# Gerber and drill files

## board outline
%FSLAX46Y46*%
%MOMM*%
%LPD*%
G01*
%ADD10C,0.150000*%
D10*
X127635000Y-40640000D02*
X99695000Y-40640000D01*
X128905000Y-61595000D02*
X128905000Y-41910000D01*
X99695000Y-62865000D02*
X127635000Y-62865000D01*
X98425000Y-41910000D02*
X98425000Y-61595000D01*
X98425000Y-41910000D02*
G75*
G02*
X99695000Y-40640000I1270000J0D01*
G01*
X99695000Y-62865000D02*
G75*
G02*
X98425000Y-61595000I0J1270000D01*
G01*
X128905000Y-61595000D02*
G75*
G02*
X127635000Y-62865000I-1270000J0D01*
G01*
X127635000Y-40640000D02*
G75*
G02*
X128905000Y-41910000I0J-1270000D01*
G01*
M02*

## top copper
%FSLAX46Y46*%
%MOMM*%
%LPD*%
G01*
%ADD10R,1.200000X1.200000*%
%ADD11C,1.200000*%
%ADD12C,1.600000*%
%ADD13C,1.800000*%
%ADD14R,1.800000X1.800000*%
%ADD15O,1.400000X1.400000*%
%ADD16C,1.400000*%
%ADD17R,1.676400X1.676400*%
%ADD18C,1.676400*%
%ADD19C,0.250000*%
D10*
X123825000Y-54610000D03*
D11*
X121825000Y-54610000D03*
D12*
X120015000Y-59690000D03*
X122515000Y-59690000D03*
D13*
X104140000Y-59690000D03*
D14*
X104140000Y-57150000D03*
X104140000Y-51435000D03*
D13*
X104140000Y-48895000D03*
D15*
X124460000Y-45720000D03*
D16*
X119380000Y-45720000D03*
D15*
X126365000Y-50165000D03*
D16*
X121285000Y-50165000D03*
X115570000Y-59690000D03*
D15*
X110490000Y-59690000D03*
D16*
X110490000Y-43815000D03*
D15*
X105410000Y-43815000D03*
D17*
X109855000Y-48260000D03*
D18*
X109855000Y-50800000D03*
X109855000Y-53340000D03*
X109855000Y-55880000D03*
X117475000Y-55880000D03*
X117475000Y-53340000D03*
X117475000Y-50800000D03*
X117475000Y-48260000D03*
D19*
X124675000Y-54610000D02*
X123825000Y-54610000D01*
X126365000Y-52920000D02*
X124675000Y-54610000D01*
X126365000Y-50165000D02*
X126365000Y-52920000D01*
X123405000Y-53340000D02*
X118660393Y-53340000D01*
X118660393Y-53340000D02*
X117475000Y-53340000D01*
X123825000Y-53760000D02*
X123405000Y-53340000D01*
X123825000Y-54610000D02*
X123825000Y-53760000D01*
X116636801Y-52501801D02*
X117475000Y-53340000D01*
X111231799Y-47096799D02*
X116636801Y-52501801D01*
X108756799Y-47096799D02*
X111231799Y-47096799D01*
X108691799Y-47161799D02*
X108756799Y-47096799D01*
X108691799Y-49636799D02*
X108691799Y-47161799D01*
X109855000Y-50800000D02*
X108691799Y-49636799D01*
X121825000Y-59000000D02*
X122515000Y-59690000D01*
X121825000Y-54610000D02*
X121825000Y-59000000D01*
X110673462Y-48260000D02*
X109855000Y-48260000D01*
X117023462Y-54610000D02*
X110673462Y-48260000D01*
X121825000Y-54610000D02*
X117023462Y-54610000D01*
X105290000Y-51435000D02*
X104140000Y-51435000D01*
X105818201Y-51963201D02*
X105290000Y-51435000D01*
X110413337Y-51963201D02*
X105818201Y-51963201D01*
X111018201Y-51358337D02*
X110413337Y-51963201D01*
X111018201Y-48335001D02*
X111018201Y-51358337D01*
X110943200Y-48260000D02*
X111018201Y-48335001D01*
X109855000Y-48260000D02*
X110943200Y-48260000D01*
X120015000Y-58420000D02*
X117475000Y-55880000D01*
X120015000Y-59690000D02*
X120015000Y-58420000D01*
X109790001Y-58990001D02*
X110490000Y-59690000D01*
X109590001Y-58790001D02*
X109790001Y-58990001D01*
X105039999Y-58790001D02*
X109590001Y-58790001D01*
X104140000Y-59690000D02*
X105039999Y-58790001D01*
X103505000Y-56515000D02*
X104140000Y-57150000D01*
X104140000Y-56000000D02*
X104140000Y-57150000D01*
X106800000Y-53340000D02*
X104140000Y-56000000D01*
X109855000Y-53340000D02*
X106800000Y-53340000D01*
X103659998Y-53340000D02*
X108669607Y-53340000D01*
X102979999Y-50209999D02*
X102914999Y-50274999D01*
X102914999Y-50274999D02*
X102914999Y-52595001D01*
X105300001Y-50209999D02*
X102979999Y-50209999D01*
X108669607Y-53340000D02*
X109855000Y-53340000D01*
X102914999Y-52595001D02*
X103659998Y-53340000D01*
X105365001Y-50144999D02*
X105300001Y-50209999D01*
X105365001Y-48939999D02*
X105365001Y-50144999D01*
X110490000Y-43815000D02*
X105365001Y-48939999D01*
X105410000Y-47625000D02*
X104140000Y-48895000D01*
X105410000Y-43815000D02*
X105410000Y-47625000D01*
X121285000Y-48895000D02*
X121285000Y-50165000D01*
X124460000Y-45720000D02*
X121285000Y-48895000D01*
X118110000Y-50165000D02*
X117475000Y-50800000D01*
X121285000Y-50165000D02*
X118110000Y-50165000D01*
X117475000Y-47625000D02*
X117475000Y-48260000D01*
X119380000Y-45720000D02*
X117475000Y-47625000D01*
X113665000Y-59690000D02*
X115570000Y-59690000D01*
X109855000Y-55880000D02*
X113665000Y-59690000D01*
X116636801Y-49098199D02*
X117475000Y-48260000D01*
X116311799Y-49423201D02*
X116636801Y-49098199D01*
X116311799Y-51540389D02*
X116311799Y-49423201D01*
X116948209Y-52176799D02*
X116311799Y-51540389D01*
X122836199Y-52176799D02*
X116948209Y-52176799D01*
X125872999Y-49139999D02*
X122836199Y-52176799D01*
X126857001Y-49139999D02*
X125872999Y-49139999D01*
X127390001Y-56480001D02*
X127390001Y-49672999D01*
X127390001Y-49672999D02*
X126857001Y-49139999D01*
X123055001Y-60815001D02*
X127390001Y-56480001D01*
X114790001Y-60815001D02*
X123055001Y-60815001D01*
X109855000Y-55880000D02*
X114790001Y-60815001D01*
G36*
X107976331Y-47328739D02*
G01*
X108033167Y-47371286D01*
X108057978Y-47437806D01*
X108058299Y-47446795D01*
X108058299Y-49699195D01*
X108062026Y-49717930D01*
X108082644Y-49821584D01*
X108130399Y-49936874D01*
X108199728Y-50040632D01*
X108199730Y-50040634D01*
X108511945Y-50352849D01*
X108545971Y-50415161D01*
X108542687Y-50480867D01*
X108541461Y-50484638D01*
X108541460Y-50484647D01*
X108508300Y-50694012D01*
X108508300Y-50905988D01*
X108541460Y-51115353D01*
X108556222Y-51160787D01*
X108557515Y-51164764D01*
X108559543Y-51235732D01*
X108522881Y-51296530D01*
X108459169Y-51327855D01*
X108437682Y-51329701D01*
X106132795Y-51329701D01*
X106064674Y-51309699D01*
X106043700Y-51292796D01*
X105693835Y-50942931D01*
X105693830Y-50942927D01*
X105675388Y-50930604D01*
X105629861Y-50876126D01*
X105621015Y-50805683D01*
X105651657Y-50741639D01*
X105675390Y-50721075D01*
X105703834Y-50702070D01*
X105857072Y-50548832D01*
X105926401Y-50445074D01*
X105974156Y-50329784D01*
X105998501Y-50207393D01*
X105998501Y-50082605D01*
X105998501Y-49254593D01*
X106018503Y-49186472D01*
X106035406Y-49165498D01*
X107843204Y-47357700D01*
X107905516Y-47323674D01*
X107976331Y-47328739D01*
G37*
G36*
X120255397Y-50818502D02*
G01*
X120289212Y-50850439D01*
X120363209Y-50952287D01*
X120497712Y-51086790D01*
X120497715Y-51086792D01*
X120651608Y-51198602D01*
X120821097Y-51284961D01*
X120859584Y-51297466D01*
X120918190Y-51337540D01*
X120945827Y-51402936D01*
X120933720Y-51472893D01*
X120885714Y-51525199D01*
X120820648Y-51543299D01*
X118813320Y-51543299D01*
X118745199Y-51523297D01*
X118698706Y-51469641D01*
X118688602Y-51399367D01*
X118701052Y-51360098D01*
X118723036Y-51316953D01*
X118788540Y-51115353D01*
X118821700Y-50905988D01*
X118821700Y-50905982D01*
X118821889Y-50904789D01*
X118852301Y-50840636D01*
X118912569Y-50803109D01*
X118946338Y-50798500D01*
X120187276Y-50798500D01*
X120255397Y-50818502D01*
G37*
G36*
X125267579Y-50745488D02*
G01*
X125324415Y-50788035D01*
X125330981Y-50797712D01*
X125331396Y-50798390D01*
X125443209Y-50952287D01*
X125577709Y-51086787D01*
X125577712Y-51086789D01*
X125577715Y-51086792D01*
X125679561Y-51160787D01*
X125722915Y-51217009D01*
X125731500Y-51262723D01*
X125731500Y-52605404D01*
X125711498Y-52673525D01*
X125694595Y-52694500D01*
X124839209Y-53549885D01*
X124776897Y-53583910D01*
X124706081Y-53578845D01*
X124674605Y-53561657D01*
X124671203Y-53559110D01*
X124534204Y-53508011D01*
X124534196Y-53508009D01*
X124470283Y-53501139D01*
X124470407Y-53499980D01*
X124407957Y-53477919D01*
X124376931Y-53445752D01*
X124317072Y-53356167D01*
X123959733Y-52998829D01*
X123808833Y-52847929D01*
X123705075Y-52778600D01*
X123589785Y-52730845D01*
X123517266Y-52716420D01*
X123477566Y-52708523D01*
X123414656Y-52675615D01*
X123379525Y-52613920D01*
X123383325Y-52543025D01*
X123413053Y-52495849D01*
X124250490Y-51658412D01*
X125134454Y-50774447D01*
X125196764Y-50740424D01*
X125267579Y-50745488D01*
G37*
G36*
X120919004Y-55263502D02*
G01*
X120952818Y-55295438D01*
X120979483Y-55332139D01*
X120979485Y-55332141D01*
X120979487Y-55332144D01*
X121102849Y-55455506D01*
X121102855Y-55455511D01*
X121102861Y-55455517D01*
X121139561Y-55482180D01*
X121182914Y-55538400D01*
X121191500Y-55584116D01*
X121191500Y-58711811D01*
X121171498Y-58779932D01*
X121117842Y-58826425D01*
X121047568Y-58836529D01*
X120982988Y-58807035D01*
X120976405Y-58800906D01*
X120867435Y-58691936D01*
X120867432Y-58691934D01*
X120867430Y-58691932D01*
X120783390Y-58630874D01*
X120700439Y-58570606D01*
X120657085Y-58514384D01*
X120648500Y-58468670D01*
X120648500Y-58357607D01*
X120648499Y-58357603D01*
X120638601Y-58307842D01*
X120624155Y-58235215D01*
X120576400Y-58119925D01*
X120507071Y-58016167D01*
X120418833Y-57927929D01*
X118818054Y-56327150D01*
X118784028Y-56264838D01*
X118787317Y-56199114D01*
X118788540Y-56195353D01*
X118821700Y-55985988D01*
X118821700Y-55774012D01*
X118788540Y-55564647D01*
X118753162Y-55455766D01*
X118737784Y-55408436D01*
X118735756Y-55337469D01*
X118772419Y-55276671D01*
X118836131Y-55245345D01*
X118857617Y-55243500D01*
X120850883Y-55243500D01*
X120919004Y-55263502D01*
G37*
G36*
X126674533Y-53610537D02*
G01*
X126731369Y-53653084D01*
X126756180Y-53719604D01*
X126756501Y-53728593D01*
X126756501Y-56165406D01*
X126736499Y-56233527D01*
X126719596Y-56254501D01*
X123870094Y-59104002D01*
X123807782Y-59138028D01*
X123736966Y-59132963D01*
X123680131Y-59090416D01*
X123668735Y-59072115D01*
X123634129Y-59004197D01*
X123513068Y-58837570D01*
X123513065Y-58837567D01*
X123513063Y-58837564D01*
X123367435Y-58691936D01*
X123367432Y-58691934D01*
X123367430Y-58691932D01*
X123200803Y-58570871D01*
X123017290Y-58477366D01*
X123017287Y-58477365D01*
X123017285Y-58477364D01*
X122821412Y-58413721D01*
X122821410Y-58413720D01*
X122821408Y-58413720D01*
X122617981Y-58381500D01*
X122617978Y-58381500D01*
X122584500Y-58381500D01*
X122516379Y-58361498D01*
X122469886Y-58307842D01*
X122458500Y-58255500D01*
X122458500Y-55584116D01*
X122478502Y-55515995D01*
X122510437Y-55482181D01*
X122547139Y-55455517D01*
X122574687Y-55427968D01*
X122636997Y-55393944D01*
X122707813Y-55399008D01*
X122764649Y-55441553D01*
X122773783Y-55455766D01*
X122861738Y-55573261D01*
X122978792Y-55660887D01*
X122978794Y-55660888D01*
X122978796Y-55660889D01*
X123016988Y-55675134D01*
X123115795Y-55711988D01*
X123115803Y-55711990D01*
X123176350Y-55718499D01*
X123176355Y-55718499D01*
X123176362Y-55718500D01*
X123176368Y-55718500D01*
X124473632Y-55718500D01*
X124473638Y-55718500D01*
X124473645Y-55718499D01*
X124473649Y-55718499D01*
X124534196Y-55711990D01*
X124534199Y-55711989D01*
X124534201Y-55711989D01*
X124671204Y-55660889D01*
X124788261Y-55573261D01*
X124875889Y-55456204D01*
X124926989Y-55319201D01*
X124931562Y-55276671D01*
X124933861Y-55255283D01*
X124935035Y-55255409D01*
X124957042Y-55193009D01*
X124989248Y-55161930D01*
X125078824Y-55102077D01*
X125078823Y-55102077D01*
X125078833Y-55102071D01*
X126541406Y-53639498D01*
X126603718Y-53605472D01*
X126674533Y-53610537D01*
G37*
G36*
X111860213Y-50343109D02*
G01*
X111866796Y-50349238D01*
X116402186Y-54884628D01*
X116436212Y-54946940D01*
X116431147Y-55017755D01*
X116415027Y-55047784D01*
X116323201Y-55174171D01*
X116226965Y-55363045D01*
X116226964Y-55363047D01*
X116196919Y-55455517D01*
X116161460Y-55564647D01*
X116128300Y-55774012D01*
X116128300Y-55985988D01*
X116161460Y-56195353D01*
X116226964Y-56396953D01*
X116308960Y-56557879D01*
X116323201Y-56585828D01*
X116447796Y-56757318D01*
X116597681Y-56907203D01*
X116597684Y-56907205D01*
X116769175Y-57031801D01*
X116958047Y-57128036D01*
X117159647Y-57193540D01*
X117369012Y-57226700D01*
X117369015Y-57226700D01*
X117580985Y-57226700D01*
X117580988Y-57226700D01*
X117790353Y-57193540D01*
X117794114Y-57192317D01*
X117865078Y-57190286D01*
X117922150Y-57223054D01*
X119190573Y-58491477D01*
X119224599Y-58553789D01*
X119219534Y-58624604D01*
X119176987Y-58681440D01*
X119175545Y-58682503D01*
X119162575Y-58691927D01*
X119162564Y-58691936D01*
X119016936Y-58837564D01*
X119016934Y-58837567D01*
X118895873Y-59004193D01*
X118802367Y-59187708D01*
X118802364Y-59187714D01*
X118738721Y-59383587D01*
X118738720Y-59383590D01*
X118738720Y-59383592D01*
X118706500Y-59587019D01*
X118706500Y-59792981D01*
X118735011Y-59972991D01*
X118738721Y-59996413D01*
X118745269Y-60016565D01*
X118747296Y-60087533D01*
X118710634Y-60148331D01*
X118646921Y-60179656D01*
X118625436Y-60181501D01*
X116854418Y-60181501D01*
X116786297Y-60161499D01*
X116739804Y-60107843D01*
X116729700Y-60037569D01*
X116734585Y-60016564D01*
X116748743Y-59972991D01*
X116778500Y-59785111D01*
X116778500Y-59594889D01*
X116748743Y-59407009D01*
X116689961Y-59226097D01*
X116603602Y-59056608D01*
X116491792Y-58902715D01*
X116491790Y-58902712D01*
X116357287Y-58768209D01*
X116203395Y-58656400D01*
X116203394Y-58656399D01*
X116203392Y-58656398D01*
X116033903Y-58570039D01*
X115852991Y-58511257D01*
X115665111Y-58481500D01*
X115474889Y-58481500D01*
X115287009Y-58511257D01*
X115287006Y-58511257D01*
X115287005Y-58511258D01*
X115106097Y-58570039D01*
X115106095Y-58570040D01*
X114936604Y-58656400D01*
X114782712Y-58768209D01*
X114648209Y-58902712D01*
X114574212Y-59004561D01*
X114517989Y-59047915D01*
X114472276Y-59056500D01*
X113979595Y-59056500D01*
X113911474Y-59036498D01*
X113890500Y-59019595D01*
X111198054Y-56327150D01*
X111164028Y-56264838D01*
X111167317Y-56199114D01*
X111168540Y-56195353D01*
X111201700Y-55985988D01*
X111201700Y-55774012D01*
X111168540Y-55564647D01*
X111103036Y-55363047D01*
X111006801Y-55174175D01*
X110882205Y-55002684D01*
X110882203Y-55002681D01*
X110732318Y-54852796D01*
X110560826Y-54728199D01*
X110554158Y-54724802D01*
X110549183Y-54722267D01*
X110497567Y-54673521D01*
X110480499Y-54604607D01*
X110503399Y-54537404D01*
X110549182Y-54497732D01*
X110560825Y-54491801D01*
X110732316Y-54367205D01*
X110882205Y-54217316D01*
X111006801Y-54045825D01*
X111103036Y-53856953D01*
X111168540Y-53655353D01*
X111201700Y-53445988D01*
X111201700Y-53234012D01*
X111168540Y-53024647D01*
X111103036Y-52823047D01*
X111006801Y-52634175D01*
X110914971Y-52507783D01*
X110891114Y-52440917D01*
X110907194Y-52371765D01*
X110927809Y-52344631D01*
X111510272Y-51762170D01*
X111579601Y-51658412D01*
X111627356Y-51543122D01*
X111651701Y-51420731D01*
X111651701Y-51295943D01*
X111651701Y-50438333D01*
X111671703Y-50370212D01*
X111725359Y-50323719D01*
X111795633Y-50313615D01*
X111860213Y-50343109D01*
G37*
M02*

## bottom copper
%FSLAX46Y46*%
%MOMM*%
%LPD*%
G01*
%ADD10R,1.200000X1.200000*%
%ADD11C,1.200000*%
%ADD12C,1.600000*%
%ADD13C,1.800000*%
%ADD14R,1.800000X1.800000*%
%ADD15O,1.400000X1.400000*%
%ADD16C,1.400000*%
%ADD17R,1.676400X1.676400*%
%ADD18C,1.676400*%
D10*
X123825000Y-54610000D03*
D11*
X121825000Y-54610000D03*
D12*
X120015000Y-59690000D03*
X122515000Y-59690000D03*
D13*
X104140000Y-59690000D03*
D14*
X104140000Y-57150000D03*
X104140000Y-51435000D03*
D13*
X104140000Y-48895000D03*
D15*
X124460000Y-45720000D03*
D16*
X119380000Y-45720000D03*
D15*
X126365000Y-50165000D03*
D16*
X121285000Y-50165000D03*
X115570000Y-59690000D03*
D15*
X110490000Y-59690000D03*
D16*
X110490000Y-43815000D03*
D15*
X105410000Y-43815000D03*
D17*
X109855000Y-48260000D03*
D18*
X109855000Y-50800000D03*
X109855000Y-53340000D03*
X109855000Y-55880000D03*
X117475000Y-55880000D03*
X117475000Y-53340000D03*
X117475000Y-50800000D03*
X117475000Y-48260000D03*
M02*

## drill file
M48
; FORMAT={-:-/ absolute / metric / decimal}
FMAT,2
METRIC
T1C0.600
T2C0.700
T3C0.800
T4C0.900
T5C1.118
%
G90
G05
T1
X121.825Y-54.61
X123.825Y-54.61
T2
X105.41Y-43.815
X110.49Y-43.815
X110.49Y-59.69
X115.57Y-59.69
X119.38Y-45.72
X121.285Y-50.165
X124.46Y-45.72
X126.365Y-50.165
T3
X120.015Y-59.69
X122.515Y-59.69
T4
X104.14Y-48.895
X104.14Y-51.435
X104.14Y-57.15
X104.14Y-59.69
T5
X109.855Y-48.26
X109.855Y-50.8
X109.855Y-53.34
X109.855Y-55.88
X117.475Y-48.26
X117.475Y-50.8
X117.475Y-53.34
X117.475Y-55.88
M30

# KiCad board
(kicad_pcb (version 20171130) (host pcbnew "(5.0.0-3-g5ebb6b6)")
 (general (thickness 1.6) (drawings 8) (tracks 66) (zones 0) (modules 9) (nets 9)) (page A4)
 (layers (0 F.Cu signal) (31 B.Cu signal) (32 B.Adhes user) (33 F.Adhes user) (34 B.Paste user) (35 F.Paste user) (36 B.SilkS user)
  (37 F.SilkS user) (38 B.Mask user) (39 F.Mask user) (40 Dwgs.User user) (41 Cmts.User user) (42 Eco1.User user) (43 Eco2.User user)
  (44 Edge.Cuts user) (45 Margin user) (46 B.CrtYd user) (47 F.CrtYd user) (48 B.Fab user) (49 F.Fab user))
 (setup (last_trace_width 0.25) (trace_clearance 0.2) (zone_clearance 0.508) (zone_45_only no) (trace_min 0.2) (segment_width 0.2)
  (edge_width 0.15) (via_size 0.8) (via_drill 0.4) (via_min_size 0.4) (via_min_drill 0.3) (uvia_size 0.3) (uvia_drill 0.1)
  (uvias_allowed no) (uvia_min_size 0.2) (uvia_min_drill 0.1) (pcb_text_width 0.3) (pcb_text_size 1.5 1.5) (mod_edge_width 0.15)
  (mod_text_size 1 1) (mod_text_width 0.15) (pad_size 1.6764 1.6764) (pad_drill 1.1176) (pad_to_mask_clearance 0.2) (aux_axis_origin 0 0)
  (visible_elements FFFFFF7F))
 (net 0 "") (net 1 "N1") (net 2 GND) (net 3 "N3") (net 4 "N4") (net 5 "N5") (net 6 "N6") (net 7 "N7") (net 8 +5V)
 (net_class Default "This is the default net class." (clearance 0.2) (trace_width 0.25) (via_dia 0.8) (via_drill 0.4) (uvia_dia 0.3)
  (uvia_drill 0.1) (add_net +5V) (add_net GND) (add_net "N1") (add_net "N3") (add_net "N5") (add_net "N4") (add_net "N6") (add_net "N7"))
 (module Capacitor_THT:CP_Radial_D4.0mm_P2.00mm (layer F.Cu) (at 123.825 54.61 180)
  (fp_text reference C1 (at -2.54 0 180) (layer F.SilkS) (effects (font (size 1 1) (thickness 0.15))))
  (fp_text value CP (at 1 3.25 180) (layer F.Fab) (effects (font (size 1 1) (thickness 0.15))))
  (pad 1 thru_hole rect (at 0 0 180) (size 1.2 1.2) (drill 0.6) (layers *.Cu *.Mask) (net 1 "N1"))
  (pad 2 thru_hole circle (at 2 0 180) (size 1.2 1.2) (drill 0.6) (layers *.Cu *.Mask) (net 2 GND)))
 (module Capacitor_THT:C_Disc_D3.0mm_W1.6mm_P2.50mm (layer F.Cu) (at 120.015 59.69)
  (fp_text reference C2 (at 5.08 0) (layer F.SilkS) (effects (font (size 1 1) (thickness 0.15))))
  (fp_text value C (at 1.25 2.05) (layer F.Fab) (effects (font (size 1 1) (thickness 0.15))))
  (pad 1 thru_hole circle (at 0 0) (size 1.6 1.6) (drill 0.8) (layers *.Cu *.Mask) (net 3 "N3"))
  (pad 2 thru_hole circle (at 2.5 0) (size 1.6 1.6) (drill 0.8) (layers *.Cu *.Mask) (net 2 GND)))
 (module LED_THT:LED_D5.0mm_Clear (layer F.Cu) (at 104.14 57.15 270)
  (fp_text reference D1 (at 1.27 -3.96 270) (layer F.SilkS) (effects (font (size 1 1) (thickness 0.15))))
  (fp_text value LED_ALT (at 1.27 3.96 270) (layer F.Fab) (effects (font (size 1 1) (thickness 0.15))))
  (pad 2 thru_hole circle (at 2.54 0 270) (size 1.8 1.8) (drill 0.9) (layers *.Cu *.Mask) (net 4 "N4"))
  (pad 1 thru_hole rect (at 0 0 270) (size 1.8 1.8) (drill 0.9) (layers *.Cu *.Mask) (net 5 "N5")))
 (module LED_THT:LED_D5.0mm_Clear (layer F.Cu) (at 104.14 51.435 90)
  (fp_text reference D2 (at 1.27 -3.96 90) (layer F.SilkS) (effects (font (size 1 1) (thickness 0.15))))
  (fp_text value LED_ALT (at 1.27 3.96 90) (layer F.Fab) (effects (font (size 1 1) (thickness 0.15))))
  (pad 1 thru_hole rect (at 0 0 90) (size 1.8 1.8) (drill 0.9) (layers *.Cu *.Mask) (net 2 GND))
  (pad 2 thru_hole circle (at 2.54 0 90) (size 1.8 1.8) (drill 0.9) (layers *.Cu *.Mask) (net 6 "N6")))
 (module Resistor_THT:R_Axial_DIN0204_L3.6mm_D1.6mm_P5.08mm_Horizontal (layer F.Cu) (at 119.38 45.72)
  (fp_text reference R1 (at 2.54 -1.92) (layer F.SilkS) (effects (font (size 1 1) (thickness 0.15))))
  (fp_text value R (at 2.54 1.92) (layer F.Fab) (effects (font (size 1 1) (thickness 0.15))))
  (pad 2 thru_hole oval (at 5.08 0) (size 1.4 1.4) (drill 0.7) (layers *.Cu *.Mask) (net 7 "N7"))
  (pad 1 thru_hole circle (at 0 0) (size 1.4 1.4) (drill 0.7) (layers *.Cu *.Mask) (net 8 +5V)))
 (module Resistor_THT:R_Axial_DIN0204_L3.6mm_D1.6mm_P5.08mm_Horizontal (layer F.Cu) (at 121.285 50.165)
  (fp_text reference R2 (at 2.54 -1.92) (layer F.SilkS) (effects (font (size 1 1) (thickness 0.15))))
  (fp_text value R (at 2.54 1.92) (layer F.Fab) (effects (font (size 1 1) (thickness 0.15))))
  (pad 2 thru_hole oval (at 5.08 0) (size 1.4 1.4) (drill 0.7) (layers *.Cu *.Mask) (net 1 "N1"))
  (pad 1 thru_hole circle (at 0 0) (size 1.4 1.4) (drill 0.7) (layers *.Cu *.Mask) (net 7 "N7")))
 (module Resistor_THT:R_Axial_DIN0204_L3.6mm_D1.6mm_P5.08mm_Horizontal (layer F.Cu) (at 115.57 59.69 180)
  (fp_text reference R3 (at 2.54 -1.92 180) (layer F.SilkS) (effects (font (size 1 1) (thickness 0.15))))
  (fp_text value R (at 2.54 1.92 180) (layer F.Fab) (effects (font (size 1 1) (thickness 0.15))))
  (pad 1 thru_hole circle (at 0 0 180) (size 1.4 1.4) (drill 0.7) (layers *.Cu *.Mask) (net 8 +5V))
  (pad 2 thru_hole oval (at 5.08 0 180) (size 1.4 1.4) (drill 0.7) (layers *.Cu *.Mask) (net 4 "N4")))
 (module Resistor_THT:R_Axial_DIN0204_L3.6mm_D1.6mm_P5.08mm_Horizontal (layer F.Cu) (at 110.49 43.815 180)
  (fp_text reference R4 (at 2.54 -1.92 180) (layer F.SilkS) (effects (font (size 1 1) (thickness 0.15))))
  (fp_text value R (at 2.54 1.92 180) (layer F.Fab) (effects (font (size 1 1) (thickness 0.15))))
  (pad 1 thru_hole circle (at 0 0 180) (size 1.4 1.4) (drill 0.7) (layers *.Cu *.Mask) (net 5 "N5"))
  (pad 2 thru_hole oval (at 5.08 0 180) (size 1.4 1.4) (drill 0.7) (layers *.Cu *.Mask) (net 6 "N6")))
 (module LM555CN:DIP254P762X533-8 (layer F.Cu) (at 117.475 55.88)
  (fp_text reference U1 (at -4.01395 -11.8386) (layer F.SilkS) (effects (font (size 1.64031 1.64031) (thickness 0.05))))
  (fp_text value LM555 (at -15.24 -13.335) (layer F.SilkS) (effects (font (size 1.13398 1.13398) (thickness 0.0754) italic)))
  (pad 1 thru_hole rect (at -7.62 -7.62) (size 1.6764 1.6764) (drill 1.1176) (layers *.Cu *.Mask) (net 2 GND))
  (pad 2 thru_hole circle (at -7.62 -5.08) (size 1.6764 1.6764) (drill 1.1176) (layers *.Cu *.Mask) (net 1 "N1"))
  (pad 3 thru_hole circle (at -7.62 -2.54) (size 1.6764 1.6764) (drill 1.1176) (layers *.Cu *.Mask) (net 5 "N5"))
  (pad 4 thru_hole circle (at -7.62 0) (size 1.6764 1.6764) (drill 1.1176) (layers *.Cu *.Mask) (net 8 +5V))
  (pad 5 thru_hole circle (at 0 0) (size 1.6764 1.6764) (drill 1.1176) (layers *.Cu *.Mask) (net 3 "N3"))
  (pad 6 thru_hole circle (at 0 -2.54) (size 1.6764 1.6764) (drill 1.1176) (layers *.Cu *.Mask) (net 1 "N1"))
  (pad 7 thru_hole circle (at 0 -5.08) (size 1.6764 1.6764) (drill 1.1176) (layers *.Cu *.Mask) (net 7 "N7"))
  (pad 8 thru_hole circle (at 0 -7.62) (size 1.6764 1.6764) (drill 1.1176) (layers *.Cu *.Mask) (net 8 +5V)))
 (gr_line (start 127.635 40.64) (end 99.695 40.64) (layer Edge.Cuts) (width 0.15))
 (gr_line (start 128.905 61.595) (end 128.905 41.91) (layer Edge.Cuts) (width 0.15))
 (gr_line (start 99.695 62.865) (end 127.635 62.865) (layer Edge.Cuts) (width 0.15))
 (gr_line (start 98.425 41.91) (end 98.425 61.595) (layer Edge.Cuts) (width 0.15))
 (gr_arc (start 99.695 41.91) (end 99.695 40.64) (angle -90) (layer Edge.Cuts) (width 0.15))
 (gr_arc (start 99.695 61.595) (end 98.425 61.595) (angle -90) (layer Edge.Cuts) (width 0.15))
 (gr_arc (start 127.635 61.595) (end 127.635 62.865) (angle -90) (layer Edge.Cuts) (width 0.15))
 (gr_arc (start 127.635 41.91) (end 128.905 41.91) (angle -90) (layer Edge.Cuts) (width 0.15))
 (segment (start 124.675 54.61) (end 123.825 54.61) (width 0.25) (layer F.Cu) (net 1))
 (segment (start 126.365 52.92) (end 124.675 54.61) (width 0.25) (layer F.Cu) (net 1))
 (segment (start 126.365 50.165) (end 126.365 52.92) (width 0.25) (layer F.Cu) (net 1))
 (segment (start 123.405 53.34) (end 118.660393 53.34) (width 0.25) (layer F.Cu) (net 1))
 (segment (start 118.660393 53.34) (end 117.475 53.34) (width 0.25) (layer F.Cu) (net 1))
 (segment (start 123.825 53.76) (end 123.405 53.34) (width 0.25) (layer F.Cu) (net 1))
 (segment (start 123.825 54.61) (end 123.825 53.76) (width 0.25) (layer F.Cu) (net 1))
 (segment (start 116.636801 52.501801) (end 117.475 53.34) (width 0.25) (layer F.Cu) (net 1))
 (segment (start 111.231799 47.096799) (end 116.636801 52.501801) (width 0.25) (layer F.Cu) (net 1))
 (segment (start 108.756799 47.096799) (end 111.231799 47.096799) (width 0.25) (layer F.Cu) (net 1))
 (segment (start 108.691799 47.161799) (end 108.756799 47.096799) (width 0.25) (layer F.Cu) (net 1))
 (segment (start 108.691799 49.636799) (end 108.691799 47.161799) (width 0.25) (layer F.Cu) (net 1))
 (segment (start 109.855 50.8) (end 108.691799 49.636799) (width 0.25) (layer F.Cu) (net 1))
 (segment (start 121.825 59) (end 122.515 59.69) (width 0.25) (layer F.Cu) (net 2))
 (segment (start 121.825 54.61) (end 121.825 59) (width 0.25) (layer F.Cu) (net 2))
 (segment (start 110.673462 48.26) (end 109.855 48.26) (width 0.25) (layer F.Cu) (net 2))
 (segment (start 117.023462 54.61) (end 110.673462 48.26) (width 0.25) (layer F.Cu) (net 2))
 (segment (start 121.825 54.61) (end 117.023462 54.61) (width 0.25) (layer F.Cu) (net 2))
 (segment (start 105.29 51.435) (end 104.14 51.435) (width 0.25) (layer F.Cu) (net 2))
 (segment (start 105.818201 51.963201) (end 105.29 51.435) (width 0.25) (layer F.Cu) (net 2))
 (segment (start 110.413337 51.963201) (end 105.818201 51.963201) (width 0.25) (layer F.Cu) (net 2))
 (segment (start 111.018201 51.358337) (end 110.413337 51.963201) (width 0.25) (layer F.Cu) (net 2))
 (segment (start 111.018201 48.335001) (end 111.018201 51.358337) (width 0.25) (layer F.Cu) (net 2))
 (segment (start 110.9432 48.26) (end 111.018201 48.335001) (width 0.25) (layer F.Cu) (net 2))
 (segment (start 109.855 48.26) (end 110.9432 48.26) (width 0.25) (layer F.Cu) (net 2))
 (segment (start 120.015 58.42) (end 117.475 55.88) (width 0.25) (layer F.Cu) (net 3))
 (segment (start 120.015 59.69) (end 120.015 58.42) (width 0.25) (layer F.Cu) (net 3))
 (segment (start 109.790001 58.990001) (end 110.49 59.69) (width 0.25) (layer F.Cu) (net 4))
 (segment (start 109.590001 58.790001) (end 109.790001 58.990001) (width 0.25) (layer F.Cu) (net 4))
 (segment (start 105.039999 58.790001) (end 109.590001 58.790001) (width 0.25) (layer F.Cu) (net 4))
 (segment (start 104.14 59.69) (end 105.039999 58.790001) (width 0.25) (layer F.Cu) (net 4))
 (segment (start 103.505 56.515) (end 104.14 57.15) (width 0.25) (layer F.Cu) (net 5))
 (segment (start 104.14 56) (end 104.14 57.15) (width 0.25) (layer F.Cu) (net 5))
 (segment (start 106.8 53.34) (end 104.14 56) (width 0.25) (layer F.Cu) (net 5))
 (segment (start 109.855 53.34) (end 106.8 53.34) (width 0.25) (layer F.Cu) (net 5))
 (segment (start 103.659998 53.34) (end 108.669607 53.34) (width 0.25) (layer F.Cu) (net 5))
 (segment (start 102.979999 50.209999) (end 102.914999 50.274999) (width 0.25) (layer F.Cu) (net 5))
 (segment (start 102.914999 50.274999) (end 102.914999 52.595001) (width 0.25) (layer F.Cu) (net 5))
 (segment (start 105.300001 50.209999) (end 102.979999 50.209999) (width 0.25) (layer F.Cu) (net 5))
 (segment (start 108.669607 53.34) (end 109.855 53.34) (width 0.25) (layer F.Cu) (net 5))
 (segment (start 102.914999 52.595001) (end 103.659998 53.34) (width 0.25) (layer F.Cu) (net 5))
 (segment (start 105.365001 50.144999) (end 105.300001 50.209999) (width 0.25) (layer F.Cu) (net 5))
 (segment (start 105.365001 48.939999) (end 105.365001 50.144999) (width 0.25) (layer F.Cu) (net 5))
 (segment (start 110.49 43.815) (end 105.365001 48.939999) (width 0.25) (layer F.Cu) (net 5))
 (segment (start 105.41 47.625) (end 104.14 48.895) (width 0.25) (layer F.Cu) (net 6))
 (segment (start 105.41 43.815) (end 105.41 47.625) (width 0.25) (layer F.Cu) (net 6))
 (segment (start 121.285 48.895) (end 121.285 50.165) (width 0.25) (layer F.Cu) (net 7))
 (segment (start 124.46 45.72) (end 121.285 48.895) (width 0.25) (layer F.Cu) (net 7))
 (segment (start 118.11 50.165) (end 117.475 50.8) (width 0.25) (layer F.Cu) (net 7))
 (segment (start 121.285 50.165) (end 118.11 50.165) (width 0.25) (layer F.Cu) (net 7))
 (segment (start 117.475 47.625) (end 117.475 48.26) (width 0.25) (layer F.Cu) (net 8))
 (segment (start 119.38 45.72) (end 117.475 47.625) (width 0.25) (layer F.Cu) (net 8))
 (segment (start 113.665 59.69) (end 115.57 59.69) (width 0.25) (layer F.Cu) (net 8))
 (segment (start 109.855 55.88) (end 113.665 59.69) (width 0.25) (layer F.Cu) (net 8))
 (segment (start 116.636801 49.098199) (end 117.475 48.26) (width 0.25) (layer F.Cu) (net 8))
 (segment (start 116.311799 49.423201) (end 116.636801 49.098199) (width 0.25) (layer F.Cu) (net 8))
 (segment (start 116.311799 51.540389) (end 116.311799 49.423201) (width 0.25) (layer F.Cu) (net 8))
 (segment (start 116.948209 52.176799) (end 116.311799 51.540389) (width 0.25) (layer F.Cu) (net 8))
 (segment (start 122.836199 52.176799) (end 116.948209 52.176799) (width 0.25) (layer F.Cu) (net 8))
 (segment (start 125.872999 49.139999) (end 122.836199 52.176799) (width 0.25) (layer F.Cu) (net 8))
 (segment (start 126.857001 49.139999) (end 125.872999 49.139999) (width 0.25) (layer F.Cu) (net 8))
 (segment (start 127.390001 56.480001) (end 127.390001 49.672999) (width 0.25) (layer F.Cu) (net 8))
 (segment (start 127.390001 49.672999) (end 126.857001 49.139999) (width 0.25) (layer F.Cu) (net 8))
 (segment (start 123.055001 60.815001) (end 127.390001 56.480001) (width 0.25) (layer F.Cu) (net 8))
 (segment (start 114.790001 60.815001) (end 123.055001 60.815001) (width 0.25) (layer F.Cu) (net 8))
 (segment (start 109.855 55.88) (end 114.790001 60.815001) (width 0.25) (layer F.Cu) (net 8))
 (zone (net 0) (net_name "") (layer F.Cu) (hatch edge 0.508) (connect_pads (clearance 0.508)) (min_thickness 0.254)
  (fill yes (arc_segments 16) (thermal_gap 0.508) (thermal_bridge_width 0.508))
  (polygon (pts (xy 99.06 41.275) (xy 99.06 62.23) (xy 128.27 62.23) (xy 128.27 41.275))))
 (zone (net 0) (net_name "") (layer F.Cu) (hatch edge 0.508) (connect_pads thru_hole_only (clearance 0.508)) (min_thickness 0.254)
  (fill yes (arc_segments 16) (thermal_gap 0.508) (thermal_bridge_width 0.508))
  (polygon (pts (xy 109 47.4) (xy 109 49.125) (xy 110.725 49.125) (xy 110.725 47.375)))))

